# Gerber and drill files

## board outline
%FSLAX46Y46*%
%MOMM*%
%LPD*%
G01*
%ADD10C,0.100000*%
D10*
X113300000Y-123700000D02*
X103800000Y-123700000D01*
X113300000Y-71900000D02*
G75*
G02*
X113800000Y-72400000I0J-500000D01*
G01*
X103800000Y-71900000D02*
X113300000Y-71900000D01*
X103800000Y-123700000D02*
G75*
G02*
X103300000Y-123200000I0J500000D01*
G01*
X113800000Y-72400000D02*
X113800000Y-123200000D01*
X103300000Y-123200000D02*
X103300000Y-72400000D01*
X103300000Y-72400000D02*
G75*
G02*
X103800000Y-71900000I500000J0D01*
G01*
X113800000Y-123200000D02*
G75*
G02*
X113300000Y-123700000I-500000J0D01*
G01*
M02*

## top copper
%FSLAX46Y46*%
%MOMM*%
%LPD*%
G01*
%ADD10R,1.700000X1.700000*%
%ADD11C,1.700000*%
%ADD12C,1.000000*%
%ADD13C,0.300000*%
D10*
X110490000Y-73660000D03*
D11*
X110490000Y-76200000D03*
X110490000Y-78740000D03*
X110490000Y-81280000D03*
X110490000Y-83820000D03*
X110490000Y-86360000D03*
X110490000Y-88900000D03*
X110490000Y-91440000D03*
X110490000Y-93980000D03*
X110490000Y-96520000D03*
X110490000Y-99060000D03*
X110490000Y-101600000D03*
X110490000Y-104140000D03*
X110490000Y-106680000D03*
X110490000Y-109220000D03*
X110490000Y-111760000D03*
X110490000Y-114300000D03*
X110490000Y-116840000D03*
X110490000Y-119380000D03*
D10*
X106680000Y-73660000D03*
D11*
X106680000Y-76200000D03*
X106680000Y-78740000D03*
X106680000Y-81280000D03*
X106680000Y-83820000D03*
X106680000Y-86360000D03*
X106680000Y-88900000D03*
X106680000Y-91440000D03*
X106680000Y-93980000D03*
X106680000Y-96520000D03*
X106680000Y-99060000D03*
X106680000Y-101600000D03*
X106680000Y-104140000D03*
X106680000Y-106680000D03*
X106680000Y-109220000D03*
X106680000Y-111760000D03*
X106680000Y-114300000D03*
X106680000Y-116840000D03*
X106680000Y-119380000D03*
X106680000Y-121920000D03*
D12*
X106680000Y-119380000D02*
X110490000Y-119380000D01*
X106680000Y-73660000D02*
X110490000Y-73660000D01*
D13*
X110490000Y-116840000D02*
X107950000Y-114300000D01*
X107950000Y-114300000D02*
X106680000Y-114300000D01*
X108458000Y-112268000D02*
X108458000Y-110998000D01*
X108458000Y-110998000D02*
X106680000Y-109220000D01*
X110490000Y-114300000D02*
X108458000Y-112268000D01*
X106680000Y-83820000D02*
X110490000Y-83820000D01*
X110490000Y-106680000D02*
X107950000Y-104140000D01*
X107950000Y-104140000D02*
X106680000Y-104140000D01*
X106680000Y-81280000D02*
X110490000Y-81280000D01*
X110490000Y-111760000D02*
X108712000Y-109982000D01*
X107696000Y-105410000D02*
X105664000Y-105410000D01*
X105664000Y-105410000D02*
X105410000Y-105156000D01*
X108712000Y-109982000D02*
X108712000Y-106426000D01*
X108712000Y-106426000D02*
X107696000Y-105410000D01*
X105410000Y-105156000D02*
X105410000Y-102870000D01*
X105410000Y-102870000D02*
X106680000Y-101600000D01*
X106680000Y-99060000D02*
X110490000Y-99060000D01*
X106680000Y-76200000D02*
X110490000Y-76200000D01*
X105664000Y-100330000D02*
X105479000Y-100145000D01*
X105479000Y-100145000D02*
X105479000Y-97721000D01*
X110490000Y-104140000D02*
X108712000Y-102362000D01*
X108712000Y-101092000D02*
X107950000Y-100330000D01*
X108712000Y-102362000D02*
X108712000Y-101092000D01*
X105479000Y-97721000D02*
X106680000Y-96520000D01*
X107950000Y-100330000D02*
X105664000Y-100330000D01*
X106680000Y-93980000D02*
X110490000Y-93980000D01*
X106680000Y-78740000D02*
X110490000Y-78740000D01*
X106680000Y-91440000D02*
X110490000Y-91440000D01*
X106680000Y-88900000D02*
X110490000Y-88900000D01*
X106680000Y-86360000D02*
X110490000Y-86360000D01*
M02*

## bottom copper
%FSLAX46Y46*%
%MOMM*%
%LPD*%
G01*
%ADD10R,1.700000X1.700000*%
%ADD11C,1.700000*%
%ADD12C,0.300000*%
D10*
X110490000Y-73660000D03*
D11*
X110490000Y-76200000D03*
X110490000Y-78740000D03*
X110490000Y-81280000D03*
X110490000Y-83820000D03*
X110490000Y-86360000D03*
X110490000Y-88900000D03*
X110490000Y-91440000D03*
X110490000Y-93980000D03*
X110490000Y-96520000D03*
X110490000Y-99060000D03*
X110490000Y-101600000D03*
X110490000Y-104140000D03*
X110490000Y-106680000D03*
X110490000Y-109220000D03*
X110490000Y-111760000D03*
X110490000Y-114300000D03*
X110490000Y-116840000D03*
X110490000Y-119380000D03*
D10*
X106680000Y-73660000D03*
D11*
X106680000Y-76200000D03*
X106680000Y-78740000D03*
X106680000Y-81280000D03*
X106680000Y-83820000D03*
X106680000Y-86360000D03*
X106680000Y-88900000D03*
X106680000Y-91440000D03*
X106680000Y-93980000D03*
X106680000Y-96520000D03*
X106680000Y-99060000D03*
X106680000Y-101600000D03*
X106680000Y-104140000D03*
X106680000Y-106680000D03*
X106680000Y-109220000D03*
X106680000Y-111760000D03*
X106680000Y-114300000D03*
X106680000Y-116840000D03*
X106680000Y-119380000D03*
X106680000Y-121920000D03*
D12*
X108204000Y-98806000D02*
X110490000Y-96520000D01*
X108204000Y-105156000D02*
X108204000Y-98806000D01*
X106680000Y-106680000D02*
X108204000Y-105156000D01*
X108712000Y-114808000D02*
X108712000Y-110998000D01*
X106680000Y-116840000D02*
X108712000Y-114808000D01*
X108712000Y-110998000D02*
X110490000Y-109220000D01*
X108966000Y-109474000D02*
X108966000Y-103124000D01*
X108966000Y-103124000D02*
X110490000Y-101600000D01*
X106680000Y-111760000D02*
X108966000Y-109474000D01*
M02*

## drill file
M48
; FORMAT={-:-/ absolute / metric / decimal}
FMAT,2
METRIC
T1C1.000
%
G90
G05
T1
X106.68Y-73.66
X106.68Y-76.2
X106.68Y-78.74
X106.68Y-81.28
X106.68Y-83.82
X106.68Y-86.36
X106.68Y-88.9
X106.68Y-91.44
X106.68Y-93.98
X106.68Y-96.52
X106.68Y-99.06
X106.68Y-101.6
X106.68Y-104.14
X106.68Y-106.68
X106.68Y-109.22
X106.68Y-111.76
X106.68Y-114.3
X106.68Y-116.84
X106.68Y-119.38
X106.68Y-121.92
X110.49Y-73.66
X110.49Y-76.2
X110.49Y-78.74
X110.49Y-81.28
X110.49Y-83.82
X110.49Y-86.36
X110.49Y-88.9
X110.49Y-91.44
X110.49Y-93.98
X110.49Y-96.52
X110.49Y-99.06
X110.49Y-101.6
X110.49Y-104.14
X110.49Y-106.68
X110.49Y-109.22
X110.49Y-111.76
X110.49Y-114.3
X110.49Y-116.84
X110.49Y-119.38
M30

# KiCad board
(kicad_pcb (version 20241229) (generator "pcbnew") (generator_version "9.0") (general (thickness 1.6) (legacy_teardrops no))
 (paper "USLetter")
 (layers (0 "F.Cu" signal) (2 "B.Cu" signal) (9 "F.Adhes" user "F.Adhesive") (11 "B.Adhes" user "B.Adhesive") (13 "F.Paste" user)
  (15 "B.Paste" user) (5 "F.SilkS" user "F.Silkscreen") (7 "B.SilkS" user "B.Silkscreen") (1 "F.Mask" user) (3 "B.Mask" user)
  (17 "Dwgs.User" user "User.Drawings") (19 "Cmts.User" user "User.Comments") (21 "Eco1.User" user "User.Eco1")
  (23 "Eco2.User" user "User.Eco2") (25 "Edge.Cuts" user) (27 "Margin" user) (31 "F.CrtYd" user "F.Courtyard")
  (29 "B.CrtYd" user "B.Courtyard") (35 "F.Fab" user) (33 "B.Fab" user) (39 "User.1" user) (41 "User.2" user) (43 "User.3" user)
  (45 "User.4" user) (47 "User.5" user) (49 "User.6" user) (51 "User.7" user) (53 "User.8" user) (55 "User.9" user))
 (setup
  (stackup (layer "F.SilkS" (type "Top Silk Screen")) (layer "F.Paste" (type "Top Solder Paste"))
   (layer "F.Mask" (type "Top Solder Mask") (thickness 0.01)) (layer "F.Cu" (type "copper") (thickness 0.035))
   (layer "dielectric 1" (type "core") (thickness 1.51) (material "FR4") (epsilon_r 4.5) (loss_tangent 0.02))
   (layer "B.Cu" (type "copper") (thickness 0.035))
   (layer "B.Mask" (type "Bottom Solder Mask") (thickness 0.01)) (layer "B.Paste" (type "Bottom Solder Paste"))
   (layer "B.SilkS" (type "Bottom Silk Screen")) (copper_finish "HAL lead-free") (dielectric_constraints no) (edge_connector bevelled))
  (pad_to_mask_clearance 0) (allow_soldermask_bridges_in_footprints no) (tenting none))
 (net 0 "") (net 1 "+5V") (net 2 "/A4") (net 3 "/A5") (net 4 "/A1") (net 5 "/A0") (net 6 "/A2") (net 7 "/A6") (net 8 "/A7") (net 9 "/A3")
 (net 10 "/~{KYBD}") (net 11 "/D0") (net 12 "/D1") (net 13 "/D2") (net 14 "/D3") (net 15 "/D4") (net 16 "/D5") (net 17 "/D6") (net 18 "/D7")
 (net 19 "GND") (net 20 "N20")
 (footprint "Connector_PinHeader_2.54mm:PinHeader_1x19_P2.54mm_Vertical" (layer "F.Cu") (at 110.49 73.66)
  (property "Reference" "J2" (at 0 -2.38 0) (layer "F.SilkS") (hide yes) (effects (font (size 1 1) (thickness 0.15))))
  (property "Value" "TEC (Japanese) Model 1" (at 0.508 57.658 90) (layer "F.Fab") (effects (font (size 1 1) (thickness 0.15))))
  (pad "1" thru_hole rect (at 0 0) (size 1.7 1.7) (drill 1) (layers "*.Cu" "*.Mask") (remove_unused_layers no) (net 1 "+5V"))
  (pad "2" thru_hole circle (at 0 2.54) (size 1.7 1.7) (drill 1) (layers "*.Cu" "*.Mask") (remove_unused_layers no) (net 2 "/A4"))
  (pad "3" thru_hole circle (at 0 5.08) (size 1.7 1.7) (drill 1) (layers "*.Cu" "*.Mask") (remove_unused_layers no) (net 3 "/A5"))
  (pad "4" thru_hole circle (at 0 7.62) (size 1.7 1.7) (drill 1) (layers "*.Cu" "*.Mask") (remove_unused_layers no) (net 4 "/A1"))
  (pad "5" thru_hole circle (at 0 10.16) (size 1.7 1.7) (drill 1) (layers "*.Cu" "*.Mask") (remove_unused_layers no) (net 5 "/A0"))
  (pad "6" thru_hole circle (at 0 12.7) (size 1.7 1.7) (drill 1) (layers "*.Cu" "*.Mask") (remove_unused_layers no) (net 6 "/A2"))
  (pad "7" thru_hole circle (at 0 15.24) (size 1.7 1.7) (drill 1) (layers "*.Cu" "*.Mask") (remove_unused_layers no) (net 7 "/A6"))
  (pad "8" thru_hole circle (at 0 17.78) (size 1.7 1.7) (drill 1) (layers "*.Cu" "*.Mask") (remove_unused_layers no) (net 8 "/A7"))
  (pad "9" thru_hole circle (at 0 20.32) (size 1.7 1.7) (drill 1) (layers "*.Cu" "*.Mask") (remove_unused_layers no) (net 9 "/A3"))
  (pad "10" thru_hole circle (at 0 22.86) (size 1.7 1.7) (drill 1) (layers "*.Cu" "*.Mask") (remove_unused_layers no) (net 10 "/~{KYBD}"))
  (pad "11" thru_hole circle (at 0 25.4) (size 1.7 1.7) (drill 1) (layers "*.Cu" "*.Mask") (remove_unused_layers no) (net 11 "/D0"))
  (pad "12" thru_hole circle (at 0 27.94) (size 1.7 1.7) (drill 1) (layers "*.Cu" "*.Mask") (remove_unused_layers no) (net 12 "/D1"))
  (pad "13" thru_hole circle (at 0 30.48) (size 1.7 1.7) (drill 1) (layers "*.Cu" "*.Mask") (remove_unused_layers no) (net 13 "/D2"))
  (pad "14" thru_hole circle (at 0 33.02) (size 1.7 1.7) (drill 1) (layers "*.Cu" "*.Mask") (remove_unused_layers no) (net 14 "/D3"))
  (pad "15" thru_hole circle (at 0 35.56) (size 1.7 1.7) (drill 1) (layers "*.Cu" "*.Mask") (remove_unused_layers no) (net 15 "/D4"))
  (pad "16" thru_hole circle (at 0 38.1) (size 1.7 1.7) (drill 1) (layers "*.Cu" "*.Mask") (remove_unused_layers no) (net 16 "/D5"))
  (pad "17" thru_hole circle (at 0 40.64) (size 1.7 1.7) (drill 1) (layers "*.Cu" "*.Mask") (remove_unused_layers no) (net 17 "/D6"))
  (pad "18" thru_hole circle (at 0 43.18) (size 1.7 1.7) (drill 1) (layers "*.Cu" "*.Mask") (remove_unused_layers no) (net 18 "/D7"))
  (pad "19" thru_hole circle (at 0 45.72) (size 1.7 1.7) (drill 1) (layers "*.Cu" "*.Mask") (remove_unused_layers no) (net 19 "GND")))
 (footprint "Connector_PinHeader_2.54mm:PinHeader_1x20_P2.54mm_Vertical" (layer "F.Cu") (at 106.68 73.66)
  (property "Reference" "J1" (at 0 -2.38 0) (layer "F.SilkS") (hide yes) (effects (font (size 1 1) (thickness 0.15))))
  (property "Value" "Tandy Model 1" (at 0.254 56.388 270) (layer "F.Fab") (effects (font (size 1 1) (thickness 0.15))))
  (pad "1" thru_hole rect (at 0 0) (size 1.7 1.7) (drill 1) (layers "*.Cu" "*.Mask") (remove_unused_layers no) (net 1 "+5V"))
  (pad "2" thru_hole circle (at 0 2.54) (size 1.7 1.7) (drill 1) (layers "*.Cu" "*.Mask") (remove_unused_layers no) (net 2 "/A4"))
  (pad "3" thru_hole circle (at 0 5.08) (size 1.7 1.7) (drill 1) (layers "*.Cu" "*.Mask") (remove_unused_layers no) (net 3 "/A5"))
  (pad "4" thru_hole circle (at 0 7.62) (size 1.7 1.7) (drill 1) (layers "*.Cu" "*.Mask") (remove_unused_layers no) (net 4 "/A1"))
  (pad "5" thru_hole circle (at 0 10.16) (size 1.7 1.7) (drill 1) (layers "*.Cu" "*.Mask") (remove_unused_layers no) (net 5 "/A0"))
  (pad "6" thru_hole circle (at 0 12.7) (size 1.7 1.7) (drill 1) (layers "*.Cu" "*.Mask") (remove_unused_layers no) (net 6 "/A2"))
  (pad "7" thru_hole circle (at 0 15.24) (size 1.7 1.7) (drill 1) (layers "*.Cu" "*.Mask") (remove_unused_layers no) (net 7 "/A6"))
  (pad "8" thru_hole circle (at 0 17.78) (size 1.7 1.7) (drill 1) (layers "*.Cu" "*.Mask") (remove_unused_layers no) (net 8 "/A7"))
  (pad "9" thru_hole circle (at 0 20.32) (size 1.7 1.7) (drill 1) (layers "*.Cu" "*.Mask") (remove_unused_layers no) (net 9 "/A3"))
  (pad "10" thru_hole circle (at 0 22.86) (size 1.7 1.7) (drill 1) (layers "*.Cu" "*.Mask") (remove_unused_layers no) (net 13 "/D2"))
  (pad "11" thru_hole circle (at 0 25.4) (size 1.7 1.7) (drill 1) (layers "*.Cu" "*.Mask") (remove_unused_layers no) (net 11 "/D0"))
  (pad "12" thru_hole circle (at 0 27.94) (size 1.7 1.7) (drill 1) (layers "*.Cu" "*.Mask") (remove_unused_layers no) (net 16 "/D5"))
  (pad "13" thru_hole circle (at 0 30.48) (size 1.7 1.7) (drill 1) (layers "*.Cu" "*.Mask") (remove_unused_layers no) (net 14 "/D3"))
  (pad "14" thru_hole circle (at 0 33.02) (size 1.7 1.7) (drill 1) (layers "*.Cu" "*.Mask") (remove_unused_layers no) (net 10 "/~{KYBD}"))
  (pad "15" thru_hole circle (at 0 35.56) (size 1.7 1.7) (drill 1) (layers "*.Cu" "*.Mask") (remove_unused_layers no) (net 17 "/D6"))
  (pad "16" thru_hole circle (at 0 38.1) (size 1.7 1.7) (drill 1) (layers "*.Cu" "*.Mask") (remove_unused_layers no) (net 12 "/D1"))
  (pad "17" thru_hole circle (at 0 40.64) (size 1.7 1.7) (drill 1) (layers "*.Cu" "*.Mask") (remove_unused_layers no) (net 18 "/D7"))
  (pad "18" thru_hole circle (at 0 43.18) (size 1.7 1.7) (drill 1) (layers "*.Cu" "*.Mask") (remove_unused_layers no) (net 15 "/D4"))
  (pad "19" thru_hole circle (at 0 45.72) (size 1.7 1.7) (drill 1) (layers "*.Cu" "*.Mask") (remove_unused_layers no) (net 19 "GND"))
  (pad "20" thru_hole circle (at 0 48.26) (size 1.7 1.7) (drill 1) (layers "*.Cu" "*.Mask") (remove_unused_layers no) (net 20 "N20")))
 (gr_line (start 113.3 123.7) (end 103.8 123.7) (stroke (width 0.1) (type default)) (layer "Edge.Cuts"))
 (gr_arc (start 113.3 71.9) (mid 113.653553 72.046447) (end 113.8 72.4) (stroke (width 0.1) (type default)) (layer "Edge.Cuts"))
 (gr_line (start 103.8 71.9) (end 113.3 71.9) (stroke (width 0.1) (type default)) (layer "Edge.Cuts"))
 (gr_arc (start 103.8 123.7) (mid 103.446447 123.553553) (end 103.3 123.2) (stroke (width 0.1) (type default)) (layer "Edge.Cuts"))
 (gr_line (start 113.8 72.4) (end 113.8 123.2) (stroke (width 0.1) (type default)) (layer "Edge.Cuts"))
 (gr_line (start 103.3 123.2) (end 103.3 72.4) (stroke (width 0.1) (type default)) (layer "Edge.Cuts"))
 (gr_arc (start 103.3 72.4) (mid 103.446447 72.046447) (end 103.8 71.9) (stroke (width 0.1) (type default)) (layer "Edge.Cuts"))
 (gr_arc (start 113.8 123.2) (mid 113.653553 123.553553) (end 113.3 123.7) (stroke (width 0.1) (type default)) (layer "Edge.Cuts"))
 (segment (start 106.68 119.38) (end 110.49 119.38) (width 1) (layer "F.Cu") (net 19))
 (segment (start 108.204 98.806) (end 110.49 96.52) (width 0.3) (layer "B.Cu") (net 10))
 (segment (start 108.204 105.156) (end 108.204 98.806) (width 0.3) (layer "B.Cu") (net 10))
 (segment (start 106.68 106.68) (end 108.204 105.156) (width 0.3) (layer "B.Cu") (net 10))
 (segment (start 106.68 73.66) (end 110.49 73.66) (width 1) (layer "F.Cu") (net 1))
 (segment (start 108.712 114.808) (end 108.712 110.998) (width 0.3) (layer "B.Cu") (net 15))
 (segment (start 106.68 116.84) (end 108.712 114.808) (width 0.3) (layer "B.Cu") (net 15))
 (segment (start 108.712 110.998) (end 110.49 109.22) (width 0.3) (layer "B.Cu") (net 15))
 (segment (start 110.49 116.84) (end 107.95 114.3) (width 0.3) (layer "F.Cu") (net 18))
 (segment (start 107.95 114.3) (end 106.68 114.3) (width 0.3) (layer "F.Cu") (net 18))
 (segment (start 108.966 109.474) (end 108.966 103.124) (width 0.3) (layer "B.Cu") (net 12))
 (segment (start 108.966 103.124) (end 110.49 101.6) (width 0.3) (layer "B.Cu") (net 12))
 (segment (start 106.68 111.76) (end 108.966 109.474) (width 0.3) (layer "B.Cu") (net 12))
 (segment (start 108.458 112.268) (end 108.458 110.998) (width 0.3) (layer "F.Cu") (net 17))
 (segment (start 108.458 110.998) (end 106.68 109.22) (width 0.3) (layer "F.Cu") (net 17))
 (segment (start 110.49 114.3) (end 108.458 112.268) (width 0.3) (layer "F.Cu") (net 17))
 (segment (start 106.68 83.82) (end 110.49 83.82) (width 0.3) (layer "F.Cu") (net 5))
 (segment (start 110.49 106.68) (end 107.95 104.14) (width 0.3) (layer "F.Cu") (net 14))
 (segment (start 107.95 104.14) (end 106.68 104.14) (width 0.3) (layer "F.Cu") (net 14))
 (segment (start 106.68 81.28) (end 110.49 81.28) (width 0.3) (layer "F.Cu") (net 4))
 (segment (start 110.49 111.76) (end 108.712 109.982) (width 0.3) (layer "F.Cu") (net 16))
 (segment (start 107.696 105.41) (end 105.664 105.41) (width 0.3) (layer "F.Cu") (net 16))
 (segment (start 105.664 105.41) (end 105.41 105.156) (width 0.3) (layer "F.Cu") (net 16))
 (segment (start 108.712 109.982) (end 108.712 106.426) (width 0.3) (layer "F.Cu") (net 16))
 (segment (start 108.712 106.426) (end 107.696 105.41) (width 0.3) (layer "F.Cu") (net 16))
 (segment (start 105.41 105.156) (end 105.41 102.87) (width 0.3) (layer "F.Cu") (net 16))
 (segment (start 105.41 102.87) (end 106.68 101.6) (width 0.3) (layer "F.Cu") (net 16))
 (segment (start 106.68 99.06) (end 110.49 99.06) (width 0.3) (layer "F.Cu") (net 11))
 (segment (start 106.68 76.2) (end 110.49 76.2) (width 0.3) (layer "F.Cu") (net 2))
 (segment (start 105.664 100.33) (end 105.479 100.145) (width 0.3) (layer "F.Cu") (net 13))
 (segment (start 105.479 100.145) (end 105.479 97.721) (width 0.3) (layer "F.Cu") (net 13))
 (segment (start 110.49 104.14) (end 108.712 102.362) (width 0.3) (layer "F.Cu") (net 13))
 (segment (start 108.712 101.092) (end 107.95 100.33) (width 0.3) (layer "F.Cu") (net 13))
 (segment (start 108.712 102.362) (end 108.712 101.092) (width 0.3) (layer "F.Cu") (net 13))
 (segment (start 105.479 97.721) (end 106.68 96.52) (width 0.3) (layer "F.Cu") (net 13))
 (segment (start 107.95 100.33) (end 105.664 100.33) (width 0.3) (layer "F.Cu") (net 13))
 (segment (start 106.68 93.98) (end 110.49 93.98) (width 0.3) (layer "F.Cu") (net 9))
 (segment (start 106.68 78.74) (end 110.49 78.74) (width 0.3) (layer "F.Cu") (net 3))
 (segment (start 106.68 91.44) (end 110.49 91.44) (width 0.3) (layer "F.Cu") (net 8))
 (segment (start 106.68 88.9) (end 110.49 88.9) (width 0.3) (layer "F.Cu") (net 7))
 (segment (start 106.68 86.36) (end 110.49 86.36) (width 0.3) (layer "F.Cu") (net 6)))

